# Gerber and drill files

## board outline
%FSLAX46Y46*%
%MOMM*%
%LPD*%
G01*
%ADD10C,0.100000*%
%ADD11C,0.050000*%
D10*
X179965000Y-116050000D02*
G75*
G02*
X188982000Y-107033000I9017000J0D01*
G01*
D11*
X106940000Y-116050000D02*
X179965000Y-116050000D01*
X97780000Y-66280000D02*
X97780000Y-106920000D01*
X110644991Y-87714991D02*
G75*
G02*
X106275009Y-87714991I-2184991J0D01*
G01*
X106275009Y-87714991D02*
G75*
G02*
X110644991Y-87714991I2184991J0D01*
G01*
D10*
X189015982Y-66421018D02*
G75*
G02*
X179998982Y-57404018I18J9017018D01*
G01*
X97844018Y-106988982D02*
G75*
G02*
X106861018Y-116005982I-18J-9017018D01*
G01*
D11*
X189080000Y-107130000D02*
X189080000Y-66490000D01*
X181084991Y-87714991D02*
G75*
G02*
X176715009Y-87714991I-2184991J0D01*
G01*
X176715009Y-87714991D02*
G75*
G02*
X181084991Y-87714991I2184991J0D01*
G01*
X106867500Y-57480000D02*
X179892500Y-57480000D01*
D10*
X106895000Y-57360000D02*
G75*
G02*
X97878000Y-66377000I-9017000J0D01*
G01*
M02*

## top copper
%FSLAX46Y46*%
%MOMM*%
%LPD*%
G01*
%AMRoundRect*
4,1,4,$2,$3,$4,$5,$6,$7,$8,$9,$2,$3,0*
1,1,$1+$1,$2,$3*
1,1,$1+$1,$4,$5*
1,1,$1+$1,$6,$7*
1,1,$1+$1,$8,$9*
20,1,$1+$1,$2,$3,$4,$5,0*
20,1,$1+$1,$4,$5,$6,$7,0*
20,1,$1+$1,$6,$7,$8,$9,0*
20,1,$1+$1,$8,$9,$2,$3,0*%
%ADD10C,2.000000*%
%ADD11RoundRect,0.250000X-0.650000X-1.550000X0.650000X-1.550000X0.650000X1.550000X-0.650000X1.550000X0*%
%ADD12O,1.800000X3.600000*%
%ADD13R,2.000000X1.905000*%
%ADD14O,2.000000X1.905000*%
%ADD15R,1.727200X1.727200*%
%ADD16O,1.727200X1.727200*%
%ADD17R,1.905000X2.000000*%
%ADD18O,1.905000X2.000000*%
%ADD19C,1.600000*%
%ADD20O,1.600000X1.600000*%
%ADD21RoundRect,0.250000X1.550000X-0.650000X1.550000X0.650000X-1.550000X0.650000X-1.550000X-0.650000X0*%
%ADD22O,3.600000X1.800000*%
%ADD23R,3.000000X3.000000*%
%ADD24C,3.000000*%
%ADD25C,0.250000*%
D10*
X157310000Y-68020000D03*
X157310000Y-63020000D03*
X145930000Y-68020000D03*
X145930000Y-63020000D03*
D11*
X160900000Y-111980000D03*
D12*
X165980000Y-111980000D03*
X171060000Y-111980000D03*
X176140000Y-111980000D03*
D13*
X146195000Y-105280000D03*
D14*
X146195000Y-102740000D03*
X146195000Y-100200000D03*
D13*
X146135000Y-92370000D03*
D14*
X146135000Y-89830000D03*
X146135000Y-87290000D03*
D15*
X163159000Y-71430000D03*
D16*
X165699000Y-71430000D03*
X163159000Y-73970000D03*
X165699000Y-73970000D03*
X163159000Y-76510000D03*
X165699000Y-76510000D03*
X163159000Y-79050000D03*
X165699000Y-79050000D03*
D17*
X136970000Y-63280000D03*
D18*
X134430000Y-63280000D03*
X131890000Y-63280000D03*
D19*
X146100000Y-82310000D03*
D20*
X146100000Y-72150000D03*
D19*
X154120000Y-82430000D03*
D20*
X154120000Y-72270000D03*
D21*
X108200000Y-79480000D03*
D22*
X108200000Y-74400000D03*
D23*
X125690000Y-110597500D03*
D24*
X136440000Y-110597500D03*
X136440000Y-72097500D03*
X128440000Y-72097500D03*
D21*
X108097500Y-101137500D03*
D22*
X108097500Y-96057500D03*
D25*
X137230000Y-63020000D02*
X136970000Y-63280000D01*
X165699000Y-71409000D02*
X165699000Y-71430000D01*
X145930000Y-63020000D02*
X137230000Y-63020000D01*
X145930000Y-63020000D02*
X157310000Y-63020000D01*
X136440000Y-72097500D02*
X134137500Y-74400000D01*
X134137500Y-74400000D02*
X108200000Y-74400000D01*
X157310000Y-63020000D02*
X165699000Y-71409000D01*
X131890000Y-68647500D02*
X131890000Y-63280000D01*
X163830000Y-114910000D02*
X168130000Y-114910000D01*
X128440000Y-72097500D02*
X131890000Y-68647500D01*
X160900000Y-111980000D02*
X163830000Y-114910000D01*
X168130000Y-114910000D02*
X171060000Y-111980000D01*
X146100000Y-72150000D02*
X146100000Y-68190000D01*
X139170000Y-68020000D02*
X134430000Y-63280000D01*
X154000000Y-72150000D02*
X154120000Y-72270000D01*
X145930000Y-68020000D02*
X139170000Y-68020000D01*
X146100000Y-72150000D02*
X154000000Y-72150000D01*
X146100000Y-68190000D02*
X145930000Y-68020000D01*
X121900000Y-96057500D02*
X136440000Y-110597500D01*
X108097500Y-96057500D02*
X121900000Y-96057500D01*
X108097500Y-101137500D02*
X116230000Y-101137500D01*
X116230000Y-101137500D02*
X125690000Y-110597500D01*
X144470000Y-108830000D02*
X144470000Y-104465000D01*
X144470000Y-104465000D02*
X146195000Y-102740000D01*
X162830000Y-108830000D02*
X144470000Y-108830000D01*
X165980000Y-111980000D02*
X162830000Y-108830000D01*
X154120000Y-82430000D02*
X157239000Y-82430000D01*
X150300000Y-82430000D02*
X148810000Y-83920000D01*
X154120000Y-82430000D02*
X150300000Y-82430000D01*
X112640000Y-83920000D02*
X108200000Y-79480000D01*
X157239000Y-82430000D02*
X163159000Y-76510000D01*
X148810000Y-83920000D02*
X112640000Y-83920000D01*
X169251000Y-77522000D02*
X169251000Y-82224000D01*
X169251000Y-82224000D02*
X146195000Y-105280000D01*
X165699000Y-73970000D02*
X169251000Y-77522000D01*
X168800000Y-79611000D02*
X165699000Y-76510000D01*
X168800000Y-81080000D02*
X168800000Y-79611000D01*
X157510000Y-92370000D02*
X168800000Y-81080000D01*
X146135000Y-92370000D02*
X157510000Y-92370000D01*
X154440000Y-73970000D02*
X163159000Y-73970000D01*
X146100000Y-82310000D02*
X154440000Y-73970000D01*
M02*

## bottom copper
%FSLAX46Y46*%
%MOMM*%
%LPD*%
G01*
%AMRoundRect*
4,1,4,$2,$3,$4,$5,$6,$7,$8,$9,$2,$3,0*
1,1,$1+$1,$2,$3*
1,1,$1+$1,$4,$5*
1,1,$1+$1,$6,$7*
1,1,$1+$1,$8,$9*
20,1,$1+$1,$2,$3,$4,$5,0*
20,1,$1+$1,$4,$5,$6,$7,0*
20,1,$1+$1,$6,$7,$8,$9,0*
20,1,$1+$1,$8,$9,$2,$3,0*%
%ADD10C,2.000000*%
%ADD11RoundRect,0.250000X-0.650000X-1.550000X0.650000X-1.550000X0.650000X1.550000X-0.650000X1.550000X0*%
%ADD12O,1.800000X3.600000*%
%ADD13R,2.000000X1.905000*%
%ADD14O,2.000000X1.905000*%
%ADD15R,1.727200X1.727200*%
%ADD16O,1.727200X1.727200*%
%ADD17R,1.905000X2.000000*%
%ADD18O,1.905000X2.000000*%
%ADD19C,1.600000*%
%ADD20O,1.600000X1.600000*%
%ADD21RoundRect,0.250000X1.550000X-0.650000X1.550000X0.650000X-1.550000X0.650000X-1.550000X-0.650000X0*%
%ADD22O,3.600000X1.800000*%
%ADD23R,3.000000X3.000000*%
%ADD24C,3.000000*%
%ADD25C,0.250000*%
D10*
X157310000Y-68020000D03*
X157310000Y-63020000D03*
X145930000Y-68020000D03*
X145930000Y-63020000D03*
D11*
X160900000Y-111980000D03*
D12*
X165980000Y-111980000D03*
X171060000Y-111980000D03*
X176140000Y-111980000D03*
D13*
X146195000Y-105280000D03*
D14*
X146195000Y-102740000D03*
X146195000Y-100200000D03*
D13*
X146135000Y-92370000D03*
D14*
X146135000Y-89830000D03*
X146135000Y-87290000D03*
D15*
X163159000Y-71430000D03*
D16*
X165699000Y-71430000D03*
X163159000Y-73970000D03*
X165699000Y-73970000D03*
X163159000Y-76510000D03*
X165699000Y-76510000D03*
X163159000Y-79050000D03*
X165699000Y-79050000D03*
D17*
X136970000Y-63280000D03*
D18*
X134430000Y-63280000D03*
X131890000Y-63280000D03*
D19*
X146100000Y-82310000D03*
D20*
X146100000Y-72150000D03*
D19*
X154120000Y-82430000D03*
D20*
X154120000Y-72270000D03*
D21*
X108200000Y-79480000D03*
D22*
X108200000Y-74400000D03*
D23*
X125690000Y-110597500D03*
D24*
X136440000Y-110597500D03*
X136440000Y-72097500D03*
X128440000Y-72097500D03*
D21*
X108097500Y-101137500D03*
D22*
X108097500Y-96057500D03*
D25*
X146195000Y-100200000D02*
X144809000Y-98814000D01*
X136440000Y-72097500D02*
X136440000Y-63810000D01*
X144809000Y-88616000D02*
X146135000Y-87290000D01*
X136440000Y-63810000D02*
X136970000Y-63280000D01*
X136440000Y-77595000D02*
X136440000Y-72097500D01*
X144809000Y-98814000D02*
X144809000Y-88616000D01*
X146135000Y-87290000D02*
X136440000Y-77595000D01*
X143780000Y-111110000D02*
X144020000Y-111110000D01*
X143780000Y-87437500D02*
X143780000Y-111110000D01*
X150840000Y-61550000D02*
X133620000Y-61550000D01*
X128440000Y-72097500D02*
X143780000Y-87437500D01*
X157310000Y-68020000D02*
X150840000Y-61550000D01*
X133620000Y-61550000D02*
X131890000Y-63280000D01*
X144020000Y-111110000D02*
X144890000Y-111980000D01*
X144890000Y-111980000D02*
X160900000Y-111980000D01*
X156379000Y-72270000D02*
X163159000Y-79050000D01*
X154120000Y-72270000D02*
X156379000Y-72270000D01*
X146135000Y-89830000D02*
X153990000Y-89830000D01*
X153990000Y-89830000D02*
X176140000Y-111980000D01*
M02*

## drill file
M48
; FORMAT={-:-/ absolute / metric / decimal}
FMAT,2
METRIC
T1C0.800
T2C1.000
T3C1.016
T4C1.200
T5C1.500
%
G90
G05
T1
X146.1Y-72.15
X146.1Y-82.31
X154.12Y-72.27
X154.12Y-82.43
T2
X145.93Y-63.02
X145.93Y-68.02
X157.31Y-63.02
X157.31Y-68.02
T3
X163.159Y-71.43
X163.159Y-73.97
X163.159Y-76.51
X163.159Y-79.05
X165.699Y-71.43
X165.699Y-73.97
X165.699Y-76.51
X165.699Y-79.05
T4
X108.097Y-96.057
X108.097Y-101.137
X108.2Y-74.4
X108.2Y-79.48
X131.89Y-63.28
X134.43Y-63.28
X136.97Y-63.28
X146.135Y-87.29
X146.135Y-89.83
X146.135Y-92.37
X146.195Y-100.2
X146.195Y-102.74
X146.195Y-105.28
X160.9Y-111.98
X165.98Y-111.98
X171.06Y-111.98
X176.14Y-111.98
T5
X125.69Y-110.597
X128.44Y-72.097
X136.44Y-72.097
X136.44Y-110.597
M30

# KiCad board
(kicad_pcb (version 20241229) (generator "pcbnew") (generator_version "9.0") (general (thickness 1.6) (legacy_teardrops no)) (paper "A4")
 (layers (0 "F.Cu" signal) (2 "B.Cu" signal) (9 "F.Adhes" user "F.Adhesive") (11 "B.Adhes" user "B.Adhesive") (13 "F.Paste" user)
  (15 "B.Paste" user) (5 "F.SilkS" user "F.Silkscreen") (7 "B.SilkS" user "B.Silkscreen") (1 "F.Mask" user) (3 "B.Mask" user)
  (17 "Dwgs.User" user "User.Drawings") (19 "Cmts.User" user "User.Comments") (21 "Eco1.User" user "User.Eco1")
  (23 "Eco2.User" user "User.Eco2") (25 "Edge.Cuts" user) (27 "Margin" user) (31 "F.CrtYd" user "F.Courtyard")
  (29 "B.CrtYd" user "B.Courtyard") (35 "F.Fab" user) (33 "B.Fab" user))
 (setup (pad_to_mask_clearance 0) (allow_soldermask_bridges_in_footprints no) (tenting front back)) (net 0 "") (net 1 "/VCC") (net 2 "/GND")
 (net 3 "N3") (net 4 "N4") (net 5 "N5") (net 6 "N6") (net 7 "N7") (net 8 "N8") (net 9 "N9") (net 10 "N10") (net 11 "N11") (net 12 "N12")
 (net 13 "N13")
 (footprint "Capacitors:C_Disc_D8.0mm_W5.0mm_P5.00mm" (layer "F.Cu") (at 157.31 68.02 90)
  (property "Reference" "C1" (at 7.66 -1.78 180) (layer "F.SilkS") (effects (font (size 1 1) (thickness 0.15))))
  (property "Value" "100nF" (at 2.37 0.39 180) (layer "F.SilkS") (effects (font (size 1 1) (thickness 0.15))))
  (pad "1" thru_hole circle (at 0 0 90) (size 2 2) (drill 1) (layers "*.Cu" "*.Mask") (remove_unused_layers no) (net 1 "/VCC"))
  (pad "2" thru_hole circle (at 5 0 90) (size 2 2) (drill 1) (layers "*.Cu" "*.Mask") (remove_unused_layers no) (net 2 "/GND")))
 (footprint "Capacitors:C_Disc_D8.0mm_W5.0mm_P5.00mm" (layer "F.Cu") (at 145.93 68.02 90)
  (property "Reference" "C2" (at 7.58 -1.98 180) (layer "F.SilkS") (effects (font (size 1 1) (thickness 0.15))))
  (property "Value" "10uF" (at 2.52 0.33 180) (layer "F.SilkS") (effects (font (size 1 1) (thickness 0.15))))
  (pad "1" thru_hole circle (at 0 0 90) (size 2 2) (drill 1) (layers "*.Cu" "*.Mask") (remove_unused_layers no) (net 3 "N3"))
  (pad "2" thru_hole circle (at 5 0 90) (size 2 2) (drill 1) (layers "*.Cu" "*.Mask") (remove_unused_layers no) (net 2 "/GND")))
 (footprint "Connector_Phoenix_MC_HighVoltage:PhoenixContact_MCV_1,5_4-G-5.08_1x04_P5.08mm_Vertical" (layer "F.Cu") (at 160.9 111.98)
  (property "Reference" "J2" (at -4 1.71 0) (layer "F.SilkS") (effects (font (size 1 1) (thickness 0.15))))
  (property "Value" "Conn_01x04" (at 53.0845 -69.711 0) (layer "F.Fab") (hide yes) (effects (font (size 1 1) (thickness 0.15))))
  (pad "1" thru_hole roundrect (at 0 0) (size 1.8 3.6) (drill 1.2) (layers "*.Cu" "*.Mask") (remove_unused_layers no)
   (roundrect_rratio 0.138889) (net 1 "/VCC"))
  (pad "2" thru_hole oval (at 5.08 0) (size 1.8 3.6) (drill 1.2) (layers "*.Cu" "*.Mask") (remove_unused_layers no) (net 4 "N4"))
  (pad "3" thru_hole oval (at 10.16 0) (size 1.8 3.6) (drill 1.2) (layers "*.Cu" "*.Mask") (remove_unused_layers no) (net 1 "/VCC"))
  (pad "4" thru_hole oval (at 15.24 0) (size 1.8 3.6) (drill 1.2) (layers "*.Cu" "*.Mask") (remove_unused_layers no) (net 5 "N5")))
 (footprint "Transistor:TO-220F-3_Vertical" (layer "F.Cu") (at 146.195 105.28 90)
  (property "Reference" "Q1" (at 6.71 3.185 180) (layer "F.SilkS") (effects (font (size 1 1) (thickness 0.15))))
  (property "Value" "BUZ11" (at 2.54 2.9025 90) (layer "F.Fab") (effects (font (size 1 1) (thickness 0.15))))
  (pad "1" thru_hole rect (at 0 0 90) (size 1.905 2) (drill 1.2) (layers "*.Cu" "*.Mask") (remove_unused_layers no) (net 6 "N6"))
  (pad "2" thru_hole oval (at 2.54 0 90) (size 1.905 2) (drill 1.2) (layers "*.Cu" "*.Mask") (remove_unused_layers no) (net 4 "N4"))
  (pad "3" thru_hole oval (at 5.08 0 90) (size 1.905 2) (drill 1.2) (layers "*.Cu" "*.Mask") (remove_unused_layers no) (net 2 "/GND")))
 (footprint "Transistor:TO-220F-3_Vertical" (layer "F.Cu") (at 146.135 92.37 90)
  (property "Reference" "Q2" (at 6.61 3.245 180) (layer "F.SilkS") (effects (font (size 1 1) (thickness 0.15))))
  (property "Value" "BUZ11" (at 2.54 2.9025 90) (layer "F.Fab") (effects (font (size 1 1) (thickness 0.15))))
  (pad "1" thru_hole rect (at 0 0 90) (size 1.905 2) (drill 1.2) (layers "*.Cu" "*.Mask") (remove_unused_layers no) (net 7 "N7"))
  (pad "2" thru_hole oval (at 2.54 0 90) (size 1.905 2) (drill 1.2) (layers "*.Cu" "*.Mask") (remove_unused_layers no) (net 5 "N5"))
  (pad "3" thru_hole oval (at 5.08 0 90) (size 1.905 2) (drill 1.2) (layers "*.Cu" "*.Mask") (remove_unused_layers no) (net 2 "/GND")))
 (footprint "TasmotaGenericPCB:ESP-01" (layer "F.Cu") (at 163.159 71.43)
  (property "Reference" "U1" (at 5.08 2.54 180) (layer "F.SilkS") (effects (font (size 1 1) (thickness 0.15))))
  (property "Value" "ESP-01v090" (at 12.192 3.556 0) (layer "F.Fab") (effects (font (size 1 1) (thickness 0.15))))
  (pad "1" thru_hole rect (at 0 0) (size 1.7272 1.7272) (drill 1.016) (layers "*.Cu" "*.Mask" "F.SilkS") (remove_unused_layers no)
   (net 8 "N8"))
  (pad "2" thru_hole oval (at 2.54 0) (size 1.7272 1.7272) (drill 1.016) (layers "*.Cu" "*.Mask" "F.SilkS") (remove_unused_layers no)
   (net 2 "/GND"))
  (pad "3" thru_hole oval (at 0 2.54) (size 1.7272 1.7272) (drill 1.016) (layers "*.Cu" "*.Mask" "F.SilkS") (remove_unused_layers no)
   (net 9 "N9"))
  (pad "4" thru_hole oval (at 2.54 2.54) (size 1.7272 1.7272) (drill 1.016) (layers "*.Cu" "*.Mask" "F.SilkS") (remove_unused_layers no)
   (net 6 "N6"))
  (pad "5" thru_hole oval (at 0 5.08) (size 1.7272 1.7272) (drill 1.016) (layers "*.Cu" "*.Mask" "F.SilkS") (remove_unused_layers no)
   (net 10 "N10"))
  (pad "6" thru_hole oval (at 2.54 5.08) (size 1.7272 1.7272) (drill 1.016) (layers "*.Cu" "*.Mask" "F.SilkS") (remove_unused_layers no)
   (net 7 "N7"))
  (pad "7" thru_hole oval (at 0 7.62) (size 1.7272 1.7272) (drill 1.016) (layers "*.Cu" "*.Mask" "F.SilkS") (remove_unused_layers no)
   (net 3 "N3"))
  (pad "8" thru_hole oval (at 2.54 7.62) (size 1.7272 1.7272) (drill 1.016) (layers "*.Cu" "*.Mask" "F.SilkS") (remove_unused_layers no)
   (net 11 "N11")))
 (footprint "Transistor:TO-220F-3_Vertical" (layer "F.Cu") (at 136.97 63.28 180)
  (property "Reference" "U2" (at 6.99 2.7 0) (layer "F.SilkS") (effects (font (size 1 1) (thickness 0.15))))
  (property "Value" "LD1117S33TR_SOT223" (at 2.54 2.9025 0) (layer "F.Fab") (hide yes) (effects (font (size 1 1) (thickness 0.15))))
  (pad "1" thru_hole rect (at 0 0 180) (size 1.905 2) (drill 1.2) (layers "*.Cu" "*.Mask") (remove_unused_layers no) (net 2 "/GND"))
  (pad "2" thru_hole oval (at 2.54 0 180) (size 1.905 2) (drill 1.2) (layers "*.Cu" "*.Mask") (remove_unused_layers no) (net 3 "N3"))
  (pad "3" thru_hole oval (at 5.08 0 180) (size 1.905 2) (drill 1.2) (layers "*.Cu" "*.Mask") (remove_unused_layers no) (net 1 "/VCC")))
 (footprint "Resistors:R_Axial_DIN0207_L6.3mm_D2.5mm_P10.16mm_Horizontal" (layer "F.Cu") (at 146.1 82.31 90)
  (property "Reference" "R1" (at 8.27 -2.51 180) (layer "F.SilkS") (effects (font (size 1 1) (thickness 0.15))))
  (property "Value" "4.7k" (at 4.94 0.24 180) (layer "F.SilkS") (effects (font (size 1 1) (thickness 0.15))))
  (pad "1" thru_hole circle (at 0 0 90) (size 1.6 1.6) (drill 0.8) (layers "*.Cu" "*.Mask") (remove_unused_layers no) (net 9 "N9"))
  (pad "2" thru_hole oval (at 10.16 0 90) (size 1.6 1.6) (drill 0.8) (layers "*.Cu" "*.Mask") (remove_unused_layers no) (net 3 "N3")))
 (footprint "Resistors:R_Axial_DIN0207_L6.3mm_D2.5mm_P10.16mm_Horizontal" (layer "F.Cu") (at 154.12 82.43 90)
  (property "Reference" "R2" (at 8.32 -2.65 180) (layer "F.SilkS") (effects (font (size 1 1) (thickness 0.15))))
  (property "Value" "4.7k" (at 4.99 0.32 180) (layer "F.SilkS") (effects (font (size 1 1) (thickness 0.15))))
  (pad "1" thru_hole circle (at 0 0 90) (size 1.6 1.6) (drill 0.8) (layers "*.Cu" "*.Mask") (remove_unused_layers no) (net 10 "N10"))
  (pad "2" thru_hole oval (at 10.16 0 90) (size 1.6 1.6) (drill 0.8) (layers "*.Cu" "*.Mask") (remove_unused_layers no) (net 3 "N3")))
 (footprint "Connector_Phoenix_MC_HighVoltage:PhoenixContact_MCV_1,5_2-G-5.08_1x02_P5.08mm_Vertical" (layer "F.Cu") (at 108.2 79.48 90)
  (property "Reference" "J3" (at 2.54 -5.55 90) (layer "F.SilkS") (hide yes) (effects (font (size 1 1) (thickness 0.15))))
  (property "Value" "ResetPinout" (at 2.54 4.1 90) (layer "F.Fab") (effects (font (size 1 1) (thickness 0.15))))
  (pad "1" thru_hole roundrect (at 0 0 90) (size 1.8 3.6) (drill 1.2) (layers "*.Cu" "*.Mask") (remove_unused_layers no)
   (roundrect_rratio 0.138889) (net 10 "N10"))
  (pad "2" thru_hole oval (at 5.08 0 90) (size 1.8 3.6) (drill 1.2) (layers "*.Cu" "*.Mask") (remove_unused_layers no) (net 2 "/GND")))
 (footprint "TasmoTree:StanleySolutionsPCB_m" (layer "F.Cu") (at 163.2 92.49)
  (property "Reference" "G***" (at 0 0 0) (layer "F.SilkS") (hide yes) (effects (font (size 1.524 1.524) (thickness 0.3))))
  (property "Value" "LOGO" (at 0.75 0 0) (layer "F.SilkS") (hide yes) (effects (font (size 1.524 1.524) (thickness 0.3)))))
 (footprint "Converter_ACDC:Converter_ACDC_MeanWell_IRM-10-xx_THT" (layer "F.Cu") (at 125.69 110.5975 90)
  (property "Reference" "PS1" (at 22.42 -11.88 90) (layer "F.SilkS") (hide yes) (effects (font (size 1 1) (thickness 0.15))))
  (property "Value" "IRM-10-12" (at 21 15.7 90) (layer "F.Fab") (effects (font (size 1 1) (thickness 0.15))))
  (pad "1" thru_hole rect (at 0 0 90) (size 3 3) (drill 1.5) (layers "*.Cu" "*.Mask") (remove_unused_layers no) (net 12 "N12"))
  (pad "2" thru_hole circle (at 0 10.75 90) (size 3 3) (drill 1.5) (layers "*.Cu" "*.Mask") (remove_unused_layers no) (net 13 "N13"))
  (pad "3" thru_hole circle (at 38.5 10.75 90) (size 3 3) (drill 1.5) (layers "*.Cu" "*.Mask") (remove_unused_layers no) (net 2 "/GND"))
  (pad "4" thru_hole circle (at 38.5 2.75 90) (size 3 3) (drill 1.5) (layers "*.Cu" "*.Mask") (remove_unused_layers no) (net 1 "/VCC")))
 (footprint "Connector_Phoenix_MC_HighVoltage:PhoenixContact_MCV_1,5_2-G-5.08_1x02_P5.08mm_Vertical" (layer "F.Cu")
  (at 108.0975 101.1375 90)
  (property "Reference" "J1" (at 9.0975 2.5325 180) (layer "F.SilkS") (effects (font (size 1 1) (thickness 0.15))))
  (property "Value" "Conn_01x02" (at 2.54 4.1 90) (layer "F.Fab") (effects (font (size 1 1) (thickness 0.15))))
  (pad "1" thru_hole roundrect (at 0 0 90) (size 1.8 3.6) (drill 1.2) (layers "*.Cu" "*.Mask") (remove_unused_layers no)
   (roundrect_rratio 0.138889) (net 12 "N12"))
  (pad "2" thru_hole oval (at 5.08 0 90) (size 1.8 3.6) (drill 1.2) (layers "*.Cu" "*.Mask") (remove_unused_layers no) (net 13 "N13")))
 (gr_arc (start 179.965 116.05) (mid 182.606018 109.674018) (end 188.982 107.033) (stroke (width 0.1) (type solid)) (layer "Edge.Cuts"))
 (gr_line (start 106.94 116.05) (end 179.965 116.05) (stroke (width 0.05) (type default)) (layer "Edge.Cuts"))
 (gr_line (start 97.78 66.28) (end 97.78 106.92) (stroke (width 0.05) (type default)) (layer "Edge.Cuts"))
 (gr_circle (center 108.46 87.714991) (end 110.238 88.984991) (stroke (width 0.05) (type solid)) (fill no) (layer "Edge.Cuts"))
 (gr_arc (start 189.015982 66.421018) (mid 182.64 63.78) (end 179.998982 57.404018) (stroke (width 0.1) (type solid)) (layer "Edge.Cuts"))
 (gr_arc (start 97.844018 106.988982) (mid 104.22 109.63) (end 106.861018 116.005982) (stroke (width 0.1) (type solid)) (layer "Edge.Cuts"))
 (gr_line (start 189.08 107.13) (end 189.08 66.49) (stroke (width 0.05) (type default)) (layer "Edge.Cuts"))
 (gr_circle (center 178.9 87.714991) (end 180.678 88.984991) (stroke (width 0.05) (type solid)) (fill no) (layer "Edge.Cuts"))
 (gr_line (start 106.8675 57.48) (end 179.8925 57.48) (stroke (width 0.05) (type default)) (layer "Edge.Cuts"))
 (gr_arc (start 106.895 57.36) (mid 104.253982 63.735982) (end 97.878 66.377) (stroke (width 0.1) (type solid)) (layer "Edge.Cuts"))
 (segment (start 137.23 63.02) (end 136.97 63.28) (width 0.25) (layer "F.Cu") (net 2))
 (segment (start 165.699 71.409) (end 165.699 71.43) (width 0.25) (layer "F.Cu") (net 2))
 (segment (start 145.93 63.02) (end 137.23 63.02) (width 0.25) (layer "F.Cu") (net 2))
 (segment (start 145.93 63.02) (end 157.31 63.02) (width 0.25) (layer "F.Cu") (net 2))
 (segment (start 136.44 72.0975) (end 134.1375 74.4) (width 0.25) (layer "F.Cu") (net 2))
 (segment (start 134.1375 74.4) (end 108.2 74.4) (width 0.25) (layer "F.Cu") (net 2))
 (segment (start 157.31 63.02) (end 165.699 71.409) (width 0.25) (layer "F.Cu") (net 2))
 (segment (start 146.195 100.2) (end 144.809 98.814) (width 0.25) (layer "B.Cu") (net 2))
 (segment (start 136.44 72.0975) (end 136.44 63.81) (width 0.25) (layer "B.Cu") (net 2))
 (segment (start 144.809 88.616) (end 146.135 87.29) (width 0.25) (layer "B.Cu") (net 2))
 (segment (start 136.44 63.81) (end 136.97 63.28) (width 0.25) (layer "B.Cu") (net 2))
 (segment (start 136.44 77.595) (end 136.44 72.0975) (width 0.25) (layer "B.Cu") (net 2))
 (segment (start 144.809 98.814) (end 144.809 88.616) (width 0.25) (layer "B.Cu") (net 2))
 (segment (start 146.135 87.29) (end 136.44 77.595) (width 0.25) (layer "B.Cu") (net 2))
 (segment (start 131.89 68.6475) (end 131.89 63.28) (width 0.25) (layer "F.Cu") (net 1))
 (segment (start 163.83 114.91) (end 168.13 114.91) (width 0.25) (layer "F.Cu") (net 1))
 (segment (start 128.44 72.0975) (end 131.89 68.6475) (width 0.25) (layer "F.Cu") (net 1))
 (segment (start 160.9 111.98) (end 163.83 114.91) (width 0.25) (layer "F.Cu") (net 1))
 (segment (start 168.13 114.91) (end 171.06 111.98) (width 0.25) (layer "F.Cu") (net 1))
 (segment (start 143.78 111.11) (end 144.02 111.11) (width 0.25) (layer "B.Cu") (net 1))
 (segment (start 143.78 87.4375) (end 143.78 111.11) (width 0.25) (layer "B.Cu") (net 1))
 (segment (start 150.84 61.55) (end 133.62 61.55) (width 0.25) (layer "B.Cu") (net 1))
 (segment (start 128.44 72.0975) (end 143.78 87.4375) (width 0.25) (layer "B.Cu") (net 1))
 (segment (start 157.31 68.02) (end 150.84 61.55) (width 0.25) (layer "B.Cu") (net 1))
 (segment (start 133.62 61.55) (end 131.89 63.28) (width 0.25) (layer "B.Cu") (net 1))
 (segment (start 144.02 111.11) (end 144.89 111.98) (width 0.25) (layer "B.Cu") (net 1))
 (segment (start 144.89 111.98) (end 160.9 111.98) (width 0.25) (layer "B.Cu") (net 1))
 (segment (start 146.1 72.15) (end 146.1 68.19) (width 0.25) (layer "F.Cu") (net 3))
 (segment (start 139.17 68.02) (end 134.43 63.28) (width 0.25) (layer "F.Cu") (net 3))
 (segment (start 154 72.15) (end 154.12 72.27) (width 0.25) (layer "F.Cu") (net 3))
 (segment (start 145.93 68.02) (end 139.17 68.02) (width 0.25) (layer "F.Cu") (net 3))
 (segment (start 146.1 72.15) (end 154 72.15) (width 0.25) (layer "F.Cu") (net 3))
 (segment (start 146.1 68.19) (end 145.93 68.02) (width 0.25) (layer "F.Cu") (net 3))
 (segment (start 156.379 72.27) (end 163.159 79.05) (width 0.25) (layer "B.Cu") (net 3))
 (segment (start 154.12 72.27) (end 156.379 72.27) (width 0.25) (layer "B.Cu") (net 3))
 (segment (start 121.9 96.0575) (end 136.44 110.5975) (width 0.25) (layer "F.Cu") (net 13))
 (segment (start 108.0975 96.0575) (end 121.9 96.0575) (width 0.25) (layer "F.Cu") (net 13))
 (segment (start 108.0975 101.1375) (end 116.23 101.1375) (width 0.25) (layer "F.Cu") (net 12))
 (segment (start 116.23 101.1375) (end 125.69 110.5975) (width 0.25) (layer "F.Cu") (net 12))
 (segment (start 146.135 89.83) (end 153.99 89.83) (width 0.25) (layer "B.Cu") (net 5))
 (segment (start 153.99 89.83) (end 176.14 111.98) (width 0.25) (layer "B.Cu") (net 5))
 (segment (start 144.47 108.83) (end 144.47 104.465) (width 0.25) (layer "F.Cu") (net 4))
 (segment (start 144.47 104.465) (end 146.195 102.74) (width 0.25) (layer "F.Cu") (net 4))
 (segment (start 162.83 108.83) (end 144.47 108.83) (width 0.25) (layer "F.Cu") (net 4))
 (segment (start 165.98 111.98) (end 162.83 108.83) (width 0.25) (layer "F.Cu") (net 4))
 (segment (start 154.12 82.43) (end 157.239 82.43) (width 0.25) (layer "F.Cu") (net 10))
 (segment (start 150.3 82.43) (end 148.81 83.92) (width 0.25) (layer "F.Cu") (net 10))
 (segment (start 154.12 82.43) (end 150.3 82.43) (width 0.25) (layer "F.Cu") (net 10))
 (segment (start 112.64 83.92) (end 108.2 79.48) (width 0.25) (layer "F.Cu") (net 10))
 (segment (start 157.239 82.43) (end 163.159 76.51) (width 0.25) (layer "F.Cu") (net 10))
 (segment (start 148.81 83.92) (end 112.64 83.92) (width 0.25) (layer "F.Cu") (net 10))
 (segment (start 169.251 77.522) (end 169.251 82.224) (width 0.25) (layer "F.Cu") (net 6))
 (segment (start 169.251 82.224) (end 146.195 105.28) (width 0.25) (layer "F.Cu") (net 6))
 (segment (start 165.699 73.97) (end 169.251 77.522) (width 0.25) (layer "F.Cu") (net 6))
 (segment (start 168.8 79.611) (end 165.699 76.51) (width 0.25) (layer "F.Cu") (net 7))
 (segment (start 168.8 81.08) (end 168.8 79.611) (width 0.25) (layer "F.Cu") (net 7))
 (segment (start 157.51 92.37) (end 168.8 81.08) (width 0.25) (layer "F.Cu") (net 7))
 (segment (start 146.135 92.37) (end 157.51 92.37) (width 0.25) (layer "F.Cu") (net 7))
 (segment (start 154.44 73.97) (end 163.159 73.97) (width 0.25) (layer "F.Cu") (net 9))
 (segment (start 146.1 82.31) (end 154.44 73.97) (width 0.25) (layer "F.Cu") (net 9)))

